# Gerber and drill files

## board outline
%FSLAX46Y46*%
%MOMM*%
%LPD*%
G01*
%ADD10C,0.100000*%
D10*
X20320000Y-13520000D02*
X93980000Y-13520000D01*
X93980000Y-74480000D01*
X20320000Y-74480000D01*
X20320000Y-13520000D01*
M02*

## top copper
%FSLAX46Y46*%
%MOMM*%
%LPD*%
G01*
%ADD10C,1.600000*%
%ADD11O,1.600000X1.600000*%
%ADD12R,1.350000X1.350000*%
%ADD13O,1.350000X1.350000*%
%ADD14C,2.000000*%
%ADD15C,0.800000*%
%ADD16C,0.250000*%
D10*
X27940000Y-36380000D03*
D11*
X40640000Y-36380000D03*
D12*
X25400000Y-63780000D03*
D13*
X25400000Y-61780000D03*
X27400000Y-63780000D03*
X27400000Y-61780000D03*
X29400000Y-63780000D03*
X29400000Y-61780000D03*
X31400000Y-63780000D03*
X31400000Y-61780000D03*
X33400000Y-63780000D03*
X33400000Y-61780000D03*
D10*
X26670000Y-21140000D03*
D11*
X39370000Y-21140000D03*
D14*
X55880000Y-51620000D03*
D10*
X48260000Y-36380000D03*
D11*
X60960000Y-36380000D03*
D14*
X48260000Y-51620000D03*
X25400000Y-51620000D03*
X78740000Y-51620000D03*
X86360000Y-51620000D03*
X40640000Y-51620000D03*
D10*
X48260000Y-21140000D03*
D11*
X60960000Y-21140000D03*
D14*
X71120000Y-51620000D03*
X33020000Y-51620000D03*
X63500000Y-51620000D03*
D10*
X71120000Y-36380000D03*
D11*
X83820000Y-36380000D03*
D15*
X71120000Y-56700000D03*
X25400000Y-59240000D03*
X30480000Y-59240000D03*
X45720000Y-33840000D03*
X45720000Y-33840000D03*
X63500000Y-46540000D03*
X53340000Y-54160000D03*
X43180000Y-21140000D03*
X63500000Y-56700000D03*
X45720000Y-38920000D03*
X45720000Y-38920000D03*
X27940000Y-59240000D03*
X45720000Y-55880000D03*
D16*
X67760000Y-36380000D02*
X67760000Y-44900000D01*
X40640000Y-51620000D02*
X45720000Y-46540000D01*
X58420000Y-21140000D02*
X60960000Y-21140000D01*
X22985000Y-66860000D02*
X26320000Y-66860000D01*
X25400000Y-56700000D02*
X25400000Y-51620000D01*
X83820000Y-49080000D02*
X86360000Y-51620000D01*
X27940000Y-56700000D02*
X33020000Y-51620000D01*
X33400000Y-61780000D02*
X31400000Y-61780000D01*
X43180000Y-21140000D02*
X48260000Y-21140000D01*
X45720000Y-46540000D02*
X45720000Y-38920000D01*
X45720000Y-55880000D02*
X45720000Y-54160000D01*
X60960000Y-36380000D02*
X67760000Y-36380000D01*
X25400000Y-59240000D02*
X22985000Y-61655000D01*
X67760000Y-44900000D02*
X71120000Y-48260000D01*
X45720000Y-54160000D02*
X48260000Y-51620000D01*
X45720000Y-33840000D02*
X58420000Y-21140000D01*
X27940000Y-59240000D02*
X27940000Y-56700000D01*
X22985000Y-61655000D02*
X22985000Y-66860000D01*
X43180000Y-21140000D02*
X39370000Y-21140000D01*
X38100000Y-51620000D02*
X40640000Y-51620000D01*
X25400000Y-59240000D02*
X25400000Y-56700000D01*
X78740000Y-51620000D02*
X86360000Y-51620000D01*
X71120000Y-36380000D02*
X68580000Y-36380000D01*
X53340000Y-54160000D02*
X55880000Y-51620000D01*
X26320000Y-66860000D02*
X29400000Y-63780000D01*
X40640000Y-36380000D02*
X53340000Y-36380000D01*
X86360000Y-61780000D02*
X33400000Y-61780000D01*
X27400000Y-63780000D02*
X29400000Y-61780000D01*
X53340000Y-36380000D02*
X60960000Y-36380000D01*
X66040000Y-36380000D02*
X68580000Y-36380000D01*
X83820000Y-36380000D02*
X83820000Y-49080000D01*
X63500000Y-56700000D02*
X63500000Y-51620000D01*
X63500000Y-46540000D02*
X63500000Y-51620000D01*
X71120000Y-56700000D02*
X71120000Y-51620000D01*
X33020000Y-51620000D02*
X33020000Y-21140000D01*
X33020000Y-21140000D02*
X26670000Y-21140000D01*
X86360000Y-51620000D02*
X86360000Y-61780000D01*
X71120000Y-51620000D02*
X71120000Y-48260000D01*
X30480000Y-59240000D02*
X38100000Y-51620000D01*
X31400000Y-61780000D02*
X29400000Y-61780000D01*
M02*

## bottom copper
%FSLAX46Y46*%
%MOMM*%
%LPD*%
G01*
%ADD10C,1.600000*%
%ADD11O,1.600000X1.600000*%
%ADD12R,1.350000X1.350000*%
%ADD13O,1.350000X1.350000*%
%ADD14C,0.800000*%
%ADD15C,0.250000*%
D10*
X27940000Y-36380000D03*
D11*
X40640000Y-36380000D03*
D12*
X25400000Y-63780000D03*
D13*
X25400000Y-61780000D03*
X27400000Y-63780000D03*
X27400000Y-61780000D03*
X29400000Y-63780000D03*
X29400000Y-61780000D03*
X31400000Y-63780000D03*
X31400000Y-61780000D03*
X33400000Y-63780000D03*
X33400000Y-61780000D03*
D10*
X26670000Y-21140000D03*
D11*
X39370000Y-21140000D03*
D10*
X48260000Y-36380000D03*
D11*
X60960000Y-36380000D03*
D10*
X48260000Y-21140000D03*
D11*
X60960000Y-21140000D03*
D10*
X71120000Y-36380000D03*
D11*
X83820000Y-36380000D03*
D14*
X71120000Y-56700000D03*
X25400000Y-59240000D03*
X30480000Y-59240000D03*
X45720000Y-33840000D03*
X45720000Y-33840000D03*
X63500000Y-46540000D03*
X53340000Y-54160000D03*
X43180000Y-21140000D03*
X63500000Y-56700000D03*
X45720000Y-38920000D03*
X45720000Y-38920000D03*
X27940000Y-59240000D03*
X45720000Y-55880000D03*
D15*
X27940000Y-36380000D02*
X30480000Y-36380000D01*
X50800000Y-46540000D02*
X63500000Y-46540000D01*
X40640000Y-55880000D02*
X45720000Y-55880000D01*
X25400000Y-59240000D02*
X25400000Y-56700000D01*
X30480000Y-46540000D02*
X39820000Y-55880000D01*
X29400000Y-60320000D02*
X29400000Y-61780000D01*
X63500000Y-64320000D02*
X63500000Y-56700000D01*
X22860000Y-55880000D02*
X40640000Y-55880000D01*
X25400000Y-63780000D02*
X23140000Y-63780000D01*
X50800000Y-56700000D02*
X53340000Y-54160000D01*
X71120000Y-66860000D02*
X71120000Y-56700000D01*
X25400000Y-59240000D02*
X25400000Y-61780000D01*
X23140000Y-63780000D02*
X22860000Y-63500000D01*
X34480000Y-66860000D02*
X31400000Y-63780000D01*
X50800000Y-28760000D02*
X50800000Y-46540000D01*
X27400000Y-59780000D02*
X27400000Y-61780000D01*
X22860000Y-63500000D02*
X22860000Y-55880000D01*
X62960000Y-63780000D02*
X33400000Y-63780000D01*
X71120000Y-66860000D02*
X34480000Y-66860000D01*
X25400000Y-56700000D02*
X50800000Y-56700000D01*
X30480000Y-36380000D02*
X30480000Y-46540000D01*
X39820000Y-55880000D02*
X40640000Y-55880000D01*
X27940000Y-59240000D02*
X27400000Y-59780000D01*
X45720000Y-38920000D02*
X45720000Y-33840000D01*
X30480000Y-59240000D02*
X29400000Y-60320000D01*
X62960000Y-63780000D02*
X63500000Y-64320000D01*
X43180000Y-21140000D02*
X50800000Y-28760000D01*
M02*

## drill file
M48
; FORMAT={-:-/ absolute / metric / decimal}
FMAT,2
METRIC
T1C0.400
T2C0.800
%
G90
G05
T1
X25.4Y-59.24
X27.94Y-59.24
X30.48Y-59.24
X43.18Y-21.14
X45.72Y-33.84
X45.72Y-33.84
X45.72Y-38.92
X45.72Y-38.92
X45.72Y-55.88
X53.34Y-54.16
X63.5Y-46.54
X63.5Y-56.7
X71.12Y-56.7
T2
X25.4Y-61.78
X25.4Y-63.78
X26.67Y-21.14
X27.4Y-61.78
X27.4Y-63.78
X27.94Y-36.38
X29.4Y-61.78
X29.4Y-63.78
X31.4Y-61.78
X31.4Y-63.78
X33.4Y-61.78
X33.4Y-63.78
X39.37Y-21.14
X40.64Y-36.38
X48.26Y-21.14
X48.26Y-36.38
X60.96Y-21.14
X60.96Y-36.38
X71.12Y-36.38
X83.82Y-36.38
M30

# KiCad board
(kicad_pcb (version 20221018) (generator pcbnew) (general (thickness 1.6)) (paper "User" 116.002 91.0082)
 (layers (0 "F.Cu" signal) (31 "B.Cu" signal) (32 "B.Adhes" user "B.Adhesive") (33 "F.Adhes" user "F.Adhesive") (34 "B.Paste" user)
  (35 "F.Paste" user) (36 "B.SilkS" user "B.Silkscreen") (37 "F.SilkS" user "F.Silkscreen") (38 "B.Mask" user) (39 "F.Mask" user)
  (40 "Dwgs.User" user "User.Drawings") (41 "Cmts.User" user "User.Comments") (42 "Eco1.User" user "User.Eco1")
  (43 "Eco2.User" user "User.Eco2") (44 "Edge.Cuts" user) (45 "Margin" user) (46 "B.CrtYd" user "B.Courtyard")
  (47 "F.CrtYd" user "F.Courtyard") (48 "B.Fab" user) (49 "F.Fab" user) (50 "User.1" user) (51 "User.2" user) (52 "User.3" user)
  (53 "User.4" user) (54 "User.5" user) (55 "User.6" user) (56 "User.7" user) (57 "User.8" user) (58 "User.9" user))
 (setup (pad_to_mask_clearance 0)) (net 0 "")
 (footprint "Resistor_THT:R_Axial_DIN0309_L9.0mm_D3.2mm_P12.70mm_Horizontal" (layer "F.Cu") (at 27.94 36.38)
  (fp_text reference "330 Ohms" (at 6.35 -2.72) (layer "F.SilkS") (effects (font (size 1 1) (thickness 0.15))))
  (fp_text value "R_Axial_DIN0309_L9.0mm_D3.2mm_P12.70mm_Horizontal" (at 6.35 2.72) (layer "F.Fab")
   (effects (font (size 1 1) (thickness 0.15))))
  (pad "1" thru_hole circle (at 0 0) (size 1.6 1.6) (drill 0.8) (layers "*.Cu" "*.Mask"))
  (pad "2" thru_hole oval (at 12.7 0) (size 1.6 1.6) (drill 0.8) (layers "*.Cu" "*.Mask")))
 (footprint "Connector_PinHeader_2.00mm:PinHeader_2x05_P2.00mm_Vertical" (layer "F.Cu") (at 25.4 63.78 90)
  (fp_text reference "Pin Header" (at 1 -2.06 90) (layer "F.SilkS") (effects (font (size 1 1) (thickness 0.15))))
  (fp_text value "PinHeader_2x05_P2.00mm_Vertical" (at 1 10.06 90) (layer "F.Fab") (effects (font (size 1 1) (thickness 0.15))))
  (pad "1" thru_hole rect (at 0 0 90) (size 1.35 1.35) (drill 0.8) (layers "*.Cu" "*.Mask"))
  (pad "2" thru_hole oval (at 2 0 90) (size 1.35 1.35) (drill 0.8) (layers "*.Cu" "*.Mask"))
  (pad "3" thru_hole oval (at 0 2 90) (size 1.35 1.35) (drill 0.8) (layers "*.Cu" "*.Mask"))
  (pad "4" thru_hole oval (at 2 2 90) (size 1.35 1.35) (drill 0.8) (layers "*.Cu" "*.Mask"))
  (pad "5" thru_hole oval (at 0 4 90) (size 1.35 1.35) (drill 0.8) (layers "*.Cu" "*.Mask"))
  (pad "6" thru_hole oval (at 2 4 90) (size 1.35 1.35) (drill 0.8) (layers "*.Cu" "*.Mask"))
  (pad "7" thru_hole oval (at 0 6 90) (size 1.35 1.35) (drill 0.8) (layers "*.Cu" "*.Mask"))
  (pad "8" thru_hole oval (at 2 6 90) (size 1.35 1.35) (drill 0.8) (layers "*.Cu" "*.Mask"))
  (pad "9" thru_hole oval (at 0 8 90) (size 1.35 1.35) (drill 0.8) (layers "*.Cu" "*.Mask"))
  (pad "10" thru_hole oval (at 2 8 90) (size 1.35 1.35) (drill 0.8) (layers "*.Cu" "*.Mask")))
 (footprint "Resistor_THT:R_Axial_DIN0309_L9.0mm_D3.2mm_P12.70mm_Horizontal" (layer "F.Cu") (at 26.67 21.14)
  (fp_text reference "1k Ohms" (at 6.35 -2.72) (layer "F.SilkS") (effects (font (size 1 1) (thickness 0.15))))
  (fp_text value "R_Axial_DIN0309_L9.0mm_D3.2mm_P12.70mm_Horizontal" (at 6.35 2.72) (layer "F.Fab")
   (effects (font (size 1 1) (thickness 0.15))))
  (pad "1" thru_hole circle (at 0 0) (size 1.6 1.6) (drill 0.8) (layers "*.Cu" "*.Mask"))
  (pad "2" thru_hole oval (at 12.7 0) (size 1.6 1.6) (drill 0.8) (layers "*.Cu" "*.Mask")))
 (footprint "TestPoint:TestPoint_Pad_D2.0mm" (layer "F.Cu") (at 55.88 51.62)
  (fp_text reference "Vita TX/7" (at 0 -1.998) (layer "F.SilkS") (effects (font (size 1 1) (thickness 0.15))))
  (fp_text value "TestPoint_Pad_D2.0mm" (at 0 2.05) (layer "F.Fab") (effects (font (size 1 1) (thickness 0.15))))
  (pad "1" smd circle (at 0 0) (size 2 2) (layers "F.Cu" "F.Mask")))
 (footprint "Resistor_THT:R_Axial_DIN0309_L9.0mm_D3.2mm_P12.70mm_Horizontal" (layer "F.Cu") (at 48.26 36.38)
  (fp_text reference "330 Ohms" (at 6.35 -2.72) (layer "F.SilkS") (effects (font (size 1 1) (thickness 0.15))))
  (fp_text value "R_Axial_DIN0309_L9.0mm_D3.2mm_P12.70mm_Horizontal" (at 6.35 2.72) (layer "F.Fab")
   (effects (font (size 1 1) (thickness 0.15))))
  (pad "1" thru_hole circle (at 0 0) (size 1.6 1.6) (drill 0.8) (layers "*.Cu" "*.Mask"))
  (pad "2" thru_hole oval (at 12.7 0) (size 1.6 1.6) (drill 0.8) (layers "*.Cu" "*.Mask")))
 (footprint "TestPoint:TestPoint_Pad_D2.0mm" (layer "F.Cu") (at 48.26 51.62)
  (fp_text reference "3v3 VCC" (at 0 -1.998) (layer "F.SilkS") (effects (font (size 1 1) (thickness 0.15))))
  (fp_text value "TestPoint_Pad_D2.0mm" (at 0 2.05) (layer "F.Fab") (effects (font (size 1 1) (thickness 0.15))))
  (pad "1" smd circle (at 0 0) (size 2 2) (layers "F.Cu" "F.Mask")))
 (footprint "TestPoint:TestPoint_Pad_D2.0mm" (layer "F.Cu") (at 25.4 51.62)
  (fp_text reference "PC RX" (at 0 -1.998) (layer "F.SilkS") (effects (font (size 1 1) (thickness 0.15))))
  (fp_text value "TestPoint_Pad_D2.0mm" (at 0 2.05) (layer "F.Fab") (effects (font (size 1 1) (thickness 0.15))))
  (pad "1" smd circle (at 0 0) (size 2 2) (layers "F.Cu" "F.Mask")))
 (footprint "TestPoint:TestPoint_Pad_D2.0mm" (layer "F.Cu") (at 78.74 51.62)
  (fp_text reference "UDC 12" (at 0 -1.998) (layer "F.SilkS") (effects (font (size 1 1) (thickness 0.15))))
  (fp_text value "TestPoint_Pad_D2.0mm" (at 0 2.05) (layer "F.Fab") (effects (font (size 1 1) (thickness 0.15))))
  (pad "1" smd circle (at 0 0) (size 2 2) (layers "F.Cu" "F.Mask")))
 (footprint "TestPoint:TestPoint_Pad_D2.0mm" (layer "F.Cu") (at 86.36 51.62)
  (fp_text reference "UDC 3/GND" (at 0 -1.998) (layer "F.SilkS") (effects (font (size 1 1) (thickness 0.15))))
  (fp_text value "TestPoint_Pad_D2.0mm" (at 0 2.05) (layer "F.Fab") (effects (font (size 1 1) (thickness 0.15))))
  (pad "1" smd circle (at 0 0) (size 2 2) (layers "F.Cu" "F.Mask")))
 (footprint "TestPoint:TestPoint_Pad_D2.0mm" (layer "F.Cu") (at 40.64 51.62)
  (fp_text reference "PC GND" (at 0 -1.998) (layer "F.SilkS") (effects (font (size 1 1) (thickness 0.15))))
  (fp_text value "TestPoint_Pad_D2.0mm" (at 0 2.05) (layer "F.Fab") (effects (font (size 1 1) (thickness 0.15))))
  (pad "1" smd circle (at 0 0) (size 2 2) (layers "F.Cu" "F.Mask")))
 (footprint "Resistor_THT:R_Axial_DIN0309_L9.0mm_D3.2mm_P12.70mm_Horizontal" (layer "F.Cu") (at 48.26 21.14)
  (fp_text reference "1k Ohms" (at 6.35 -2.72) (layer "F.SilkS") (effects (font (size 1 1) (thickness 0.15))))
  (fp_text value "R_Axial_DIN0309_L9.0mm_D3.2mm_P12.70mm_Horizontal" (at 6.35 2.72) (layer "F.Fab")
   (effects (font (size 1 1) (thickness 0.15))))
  (pad "1" thru_hole circle (at 0 0) (size 1.6 1.6) (drill 0.8) (layers "*.Cu" "*.Mask"))
  (pad "2" thru_hole oval (at 12.7 0) (size 1.6 1.6) (drill 0.8) (layers "*.Cu" "*.Mask")))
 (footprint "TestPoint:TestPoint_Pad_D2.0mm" (layer "F.Cu") (at 71.12 51.62)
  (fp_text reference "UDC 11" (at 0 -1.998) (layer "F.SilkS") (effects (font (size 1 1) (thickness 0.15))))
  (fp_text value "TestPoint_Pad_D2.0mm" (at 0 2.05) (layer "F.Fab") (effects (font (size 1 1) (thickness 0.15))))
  (pad "1" smd circle (at 0 0) (size 2 2) (layers "F.Cu" "F.Mask")))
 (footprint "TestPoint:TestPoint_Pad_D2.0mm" (layer "F.Cu") (at 33.02 51.62)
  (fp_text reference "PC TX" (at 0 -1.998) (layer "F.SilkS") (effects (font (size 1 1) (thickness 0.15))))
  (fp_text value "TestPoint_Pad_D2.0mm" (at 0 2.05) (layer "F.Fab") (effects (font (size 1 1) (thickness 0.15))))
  (pad "1" smd circle (at 0 0) (size 2 2) (layers "F.Cu" "F.Mask")))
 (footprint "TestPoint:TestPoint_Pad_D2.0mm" (layer "F.Cu") (at 63.5 51.62)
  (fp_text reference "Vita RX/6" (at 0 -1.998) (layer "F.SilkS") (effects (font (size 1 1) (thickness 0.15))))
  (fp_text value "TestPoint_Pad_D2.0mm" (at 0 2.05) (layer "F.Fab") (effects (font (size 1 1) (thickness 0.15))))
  (pad "1" smd circle (at 0 0) (size 2 2) (layers "F.Cu" "F.Mask")))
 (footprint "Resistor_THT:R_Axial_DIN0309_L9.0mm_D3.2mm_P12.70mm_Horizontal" (layer "F.Cu") (at 71.12 36.38)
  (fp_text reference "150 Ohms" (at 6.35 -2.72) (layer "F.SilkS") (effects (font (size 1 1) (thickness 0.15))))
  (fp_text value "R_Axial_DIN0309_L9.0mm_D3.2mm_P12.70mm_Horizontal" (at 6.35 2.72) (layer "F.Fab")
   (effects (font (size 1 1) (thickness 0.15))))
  (pad "1" thru_hole circle (at 0 0) (size 1.6 1.6) (drill 0.8) (layers "*.Cu" "*.Mask"))
  (pad "2" thru_hole oval (at 12.7 0) (size 1.6 1.6) (drill 0.8) (layers "*.Cu" "*.Mask")))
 (gr_rect (start 20.32 13.52) (end 93.98 74.48) (stroke (width 0.1) (type default)) (fill none) (layer "Edge.Cuts"))
 (segment (start 67.76 36.38) (end 67.76 44.9) (width 0.25) (layer "F.Cu") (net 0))
 (segment (start 40.64 51.62) (end 45.72 46.54) (width 0.25) (layer "F.Cu") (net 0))
 (segment (start 58.42 21.14) (end 60.96 21.14) (width 0.25) (layer "F.Cu") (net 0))
 (segment (start 22.985 66.86) (end 26.32 66.86) (width 0.25) (layer "F.Cu") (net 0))
 (segment (start 25.4 56.7) (end 25.4 51.62) (width 0.25) (layer "F.Cu") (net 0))
 (segment (start 83.82 49.08) (end 86.36 51.62) (width 0.25) (layer "F.Cu") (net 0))
 (segment (start 27.94 56.7) (end 33.02 51.62) (width 0.25) (layer "F.Cu") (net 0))
 (segment (start 33.4 61.78) (end 31.4 61.78) (width 0.25) (layer "F.Cu") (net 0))
 (segment (start 43.18 21.14) (end 48.26 21.14) (width 0.25) (layer "F.Cu") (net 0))
 (segment (start 45.72 46.54) (end 45.72 38.92) (width 0.25) (layer "F.Cu") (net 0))
 (segment (start 45.72 55.88) (end 45.72 54.16) (width 0.25) (layer "F.Cu") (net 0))
 (segment (start 60.96 36.38) (end 67.76 36.38) (width 0.25) (layer "F.Cu") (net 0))
 (segment (start 25.4 59.24) (end 22.985 61.655) (width 0.25) (layer "F.Cu") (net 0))
 (segment (start 67.76 44.9) (end 71.12 48.26) (width 0.25) (layer "F.Cu") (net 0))
 (segment (start 45.72 54.16) (end 48.26 51.62) (width 0.25) (layer "F.Cu") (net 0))
 (segment (start 45.72 33.84) (end 58.42 21.14) (width 0.25) (layer "F.Cu") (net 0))
 (segment (start 27.94 59.24) (end 27.94 56.7) (width 0.25) (layer "F.Cu") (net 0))
 (segment (start 22.985 61.655) (end 22.985 66.86) (width 0.25) (layer "F.Cu") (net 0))
 (segment (start 43.18 21.14) (end 39.37 21.14) (width 0.25) (layer "F.Cu") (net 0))
 (segment (start 38.1 51.62) (end 40.64 51.62) (width 0.25) (layer "F.Cu") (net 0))
 (segment (start 25.4 59.24) (end 25.4 56.7) (width 0.25) (layer "F.Cu") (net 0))
 (segment (start 78.74 51.62) (end 86.36 51.62) (width 0.25) (layer "F.Cu") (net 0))
 (segment (start 71.12 36.38) (end 68.58 36.38) (width 0.25) (layer "F.Cu") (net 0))
 (segment (start 53.34 54.16) (end 55.88 51.62) (width 0.25) (layer "F.Cu") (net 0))
 (segment (start 26.32 66.86) (end 29.4 63.78) (width 0.25) (layer "F.Cu") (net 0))
 (segment (start 40.64 36.38) (end 53.34 36.38) (width 0.25) (layer "F.Cu") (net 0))
 (segment (start 86.36 61.78) (end 33.4 61.78) (width 0.25) (layer "F.Cu") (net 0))
 (segment (start 27.4 63.78) (end 29.4 61.78) (width 0.25) (layer "F.Cu") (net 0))
 (segment (start 53.34 36.38) (end 60.96 36.38) (width 0.25) (layer "F.Cu") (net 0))
 (segment (start 66.04 36.38) (end 68.58 36.38) (width 0.25) (layer "F.Cu") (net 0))
 (segment (start 83.82 36.38) (end 83.82 49.08) (width 0.25) (layer "F.Cu") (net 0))
 (segment (start 63.5 56.7) (end 63.5 51.62) (width 0.25) (layer "F.Cu") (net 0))
 (segment (start 63.5 46.54) (end 63.5 51.62) (width 0.25) (layer "F.Cu") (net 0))
 (segment (start 71.12 56.7) (end 71.12 51.62) (width 0.25) (layer "F.Cu") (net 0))
 (segment (start 33.02 51.62) (end 33.02 21.14) (width 0.25) (layer "F.Cu") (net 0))
 (segment (start 33.02 21.14) (end 26.67 21.14) (width 0.25) (layer "F.Cu") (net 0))
 (segment (start 86.36 51.62) (end 86.36 61.78) (width 0.25) (layer "F.Cu") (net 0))
 (segment (start 71.12 51.62) (end 71.12 48.26) (width 0.25) (layer "F.Cu") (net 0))
 (segment (start 30.48 59.24) (end 38.1 51.62) (width 0.25) (layer "F.Cu") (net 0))
 (segment (start 31.4 61.78) (end 29.4 61.78) (width 0.25) (layer "F.Cu") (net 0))
 (via (at 71.12 56.7) (size 0.8) (drill 0.4) (layers "F.Cu" "B.Cu") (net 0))
 (via (at 25.4 59.24) (size 0.8) (drill 0.4) (layers "F.Cu" "B.Cu") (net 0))
 (via (at 30.48 59.24) (size 0.8) (drill 0.4) (layers "F.Cu" "B.Cu") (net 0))
 (via (at 45.72 33.84) (size 0.8) (drill 0.4) (layers "F.Cu" "B.Cu") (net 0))
 (via (at 45.72 33.84) (size 0.8) (drill 0.4) (layers "F.Cu" "B.Cu") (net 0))
 (via (at 63.5 46.54) (size 0.8) (drill 0.4) (layers "F.Cu" "B.Cu") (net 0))
 (via (at 53.34 54.16) (size 0.8) (drill 0.4) (layers "F.Cu" "B.Cu") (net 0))
 (via (at 43.18 21.14) (size 0.8) (drill 0.4) (layers "F.Cu" "B.Cu") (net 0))
 (via (at 63.5 56.7) (size 0.8) (drill 0.4) (layers "F.Cu" "B.Cu") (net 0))
 (via (at 45.72 38.92) (size 0.8) (drill 0.4) (layers "F.Cu" "B.Cu") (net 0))
 (via (at 45.72 38.92) (size 0.8) (drill 0.4) (layers "F.Cu" "B.Cu") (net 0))
 (via (at 27.94 59.24) (size 0.8) (drill 0.4) (layers "F.Cu" "B.Cu") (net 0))
 (via (at 45.72 55.88) (size 0.8) (drill 0.4) (layers "F.Cu" "B.Cu") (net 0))
 (segment (start 27.94 36.38) (end 30.48 36.38) (width 0.25) (layer "B.Cu") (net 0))
 (segment (start 50.8 46.54) (end 63.5 46.54) (width 0.25) (layer "B.Cu") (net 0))
 (segment (start 40.64 55.88) (end 45.72 55.88) (width 0.25) (layer "B.Cu") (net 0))
 (segment (start 25.4 59.24) (end 25.4 56.7) (width 0.25) (layer "B.Cu") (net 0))
 (segment (start 30.48 46.54) (end 39.82 55.88) (width 0.25) (layer "B.Cu") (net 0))
 (segment (start 29.4 60.32) (end 29.4 61.78) (width 0.25) (layer "B.Cu") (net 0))
 (segment (start 63.5 64.32) (end 63.5 56.7) (width 0.25) (layer "B.Cu") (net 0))
 (segment (start 22.86 55.88) (end 40.64 55.88) (width 0.25) (layer "B.Cu") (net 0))
 (segment (start 25.4 63.78) (end 23.14 63.78) (width 0.25) (layer "B.Cu") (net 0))
 (segment (start 50.8 56.7) (end 53.34 54.16) (width 0.25) (layer "B.Cu") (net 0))
 (segment (start 71.12 66.86) (end 71.12 56.7) (width 0.25) (layer "B.Cu") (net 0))
 (segment (start 25.4 59.24) (end 25.4 61.78) (width 0.25) (layer "B.Cu") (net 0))
 (segment (start 23.14 63.78) (end 22.86 63.5) (width 0.25) (layer "B.Cu") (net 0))
 (segment (start 34.48 66.86) (end 31.4 63.78) (width 0.25) (layer "B.Cu") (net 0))
 (segment (start 50.8 28.76) (end 50.8 46.54) (width 0.25) (layer "B.Cu") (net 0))
 (segment (start 27.4 59.78) (end 27.4 61.78) (width 0.25) (layer "B.Cu") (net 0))
 (segment (start 22.86 63.5) (end 22.86 55.88) (width 0.25) (layer "B.Cu") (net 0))
 (segment (start 62.96 63.78) (end 33.4 63.78) (width 0.25) (layer "B.Cu") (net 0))
 (segment (start 71.12 66.86) (end 34.48 66.86) (width 0.25) (layer "B.Cu") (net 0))
 (segment (start 25.4 56.7) (end 50.8 56.7) (width 0.25) (layer "B.Cu") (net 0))
 (segment (start 30.48 36.38) (end 30.48 46.54) (width 0.25) (layer "B.Cu") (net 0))
 (segment (start 39.82 55.88) (end 40.64 55.88) (width 0.25) (layer "B.Cu") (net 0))
 (segment (start 27.94 59.24) (end 27.4 59.78) (width 0.25) (layer "B.Cu") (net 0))
 (segment (start 45.72 38.92) (end 45.72 33.84) (width 0.25) (layer "B.Cu") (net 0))
 (segment (start 30.48 59.24) (end 29.4 60.32) (width 0.25) (layer "B.Cu") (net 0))
 (segment (start 62.96 63.78) (end 63.5 64.32) (width 0.25) (layer "B.Cu") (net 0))
 (segment (start 43.18 21.14) (end 50.8 28.76) (width 0.25) (layer "B.Cu") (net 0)))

